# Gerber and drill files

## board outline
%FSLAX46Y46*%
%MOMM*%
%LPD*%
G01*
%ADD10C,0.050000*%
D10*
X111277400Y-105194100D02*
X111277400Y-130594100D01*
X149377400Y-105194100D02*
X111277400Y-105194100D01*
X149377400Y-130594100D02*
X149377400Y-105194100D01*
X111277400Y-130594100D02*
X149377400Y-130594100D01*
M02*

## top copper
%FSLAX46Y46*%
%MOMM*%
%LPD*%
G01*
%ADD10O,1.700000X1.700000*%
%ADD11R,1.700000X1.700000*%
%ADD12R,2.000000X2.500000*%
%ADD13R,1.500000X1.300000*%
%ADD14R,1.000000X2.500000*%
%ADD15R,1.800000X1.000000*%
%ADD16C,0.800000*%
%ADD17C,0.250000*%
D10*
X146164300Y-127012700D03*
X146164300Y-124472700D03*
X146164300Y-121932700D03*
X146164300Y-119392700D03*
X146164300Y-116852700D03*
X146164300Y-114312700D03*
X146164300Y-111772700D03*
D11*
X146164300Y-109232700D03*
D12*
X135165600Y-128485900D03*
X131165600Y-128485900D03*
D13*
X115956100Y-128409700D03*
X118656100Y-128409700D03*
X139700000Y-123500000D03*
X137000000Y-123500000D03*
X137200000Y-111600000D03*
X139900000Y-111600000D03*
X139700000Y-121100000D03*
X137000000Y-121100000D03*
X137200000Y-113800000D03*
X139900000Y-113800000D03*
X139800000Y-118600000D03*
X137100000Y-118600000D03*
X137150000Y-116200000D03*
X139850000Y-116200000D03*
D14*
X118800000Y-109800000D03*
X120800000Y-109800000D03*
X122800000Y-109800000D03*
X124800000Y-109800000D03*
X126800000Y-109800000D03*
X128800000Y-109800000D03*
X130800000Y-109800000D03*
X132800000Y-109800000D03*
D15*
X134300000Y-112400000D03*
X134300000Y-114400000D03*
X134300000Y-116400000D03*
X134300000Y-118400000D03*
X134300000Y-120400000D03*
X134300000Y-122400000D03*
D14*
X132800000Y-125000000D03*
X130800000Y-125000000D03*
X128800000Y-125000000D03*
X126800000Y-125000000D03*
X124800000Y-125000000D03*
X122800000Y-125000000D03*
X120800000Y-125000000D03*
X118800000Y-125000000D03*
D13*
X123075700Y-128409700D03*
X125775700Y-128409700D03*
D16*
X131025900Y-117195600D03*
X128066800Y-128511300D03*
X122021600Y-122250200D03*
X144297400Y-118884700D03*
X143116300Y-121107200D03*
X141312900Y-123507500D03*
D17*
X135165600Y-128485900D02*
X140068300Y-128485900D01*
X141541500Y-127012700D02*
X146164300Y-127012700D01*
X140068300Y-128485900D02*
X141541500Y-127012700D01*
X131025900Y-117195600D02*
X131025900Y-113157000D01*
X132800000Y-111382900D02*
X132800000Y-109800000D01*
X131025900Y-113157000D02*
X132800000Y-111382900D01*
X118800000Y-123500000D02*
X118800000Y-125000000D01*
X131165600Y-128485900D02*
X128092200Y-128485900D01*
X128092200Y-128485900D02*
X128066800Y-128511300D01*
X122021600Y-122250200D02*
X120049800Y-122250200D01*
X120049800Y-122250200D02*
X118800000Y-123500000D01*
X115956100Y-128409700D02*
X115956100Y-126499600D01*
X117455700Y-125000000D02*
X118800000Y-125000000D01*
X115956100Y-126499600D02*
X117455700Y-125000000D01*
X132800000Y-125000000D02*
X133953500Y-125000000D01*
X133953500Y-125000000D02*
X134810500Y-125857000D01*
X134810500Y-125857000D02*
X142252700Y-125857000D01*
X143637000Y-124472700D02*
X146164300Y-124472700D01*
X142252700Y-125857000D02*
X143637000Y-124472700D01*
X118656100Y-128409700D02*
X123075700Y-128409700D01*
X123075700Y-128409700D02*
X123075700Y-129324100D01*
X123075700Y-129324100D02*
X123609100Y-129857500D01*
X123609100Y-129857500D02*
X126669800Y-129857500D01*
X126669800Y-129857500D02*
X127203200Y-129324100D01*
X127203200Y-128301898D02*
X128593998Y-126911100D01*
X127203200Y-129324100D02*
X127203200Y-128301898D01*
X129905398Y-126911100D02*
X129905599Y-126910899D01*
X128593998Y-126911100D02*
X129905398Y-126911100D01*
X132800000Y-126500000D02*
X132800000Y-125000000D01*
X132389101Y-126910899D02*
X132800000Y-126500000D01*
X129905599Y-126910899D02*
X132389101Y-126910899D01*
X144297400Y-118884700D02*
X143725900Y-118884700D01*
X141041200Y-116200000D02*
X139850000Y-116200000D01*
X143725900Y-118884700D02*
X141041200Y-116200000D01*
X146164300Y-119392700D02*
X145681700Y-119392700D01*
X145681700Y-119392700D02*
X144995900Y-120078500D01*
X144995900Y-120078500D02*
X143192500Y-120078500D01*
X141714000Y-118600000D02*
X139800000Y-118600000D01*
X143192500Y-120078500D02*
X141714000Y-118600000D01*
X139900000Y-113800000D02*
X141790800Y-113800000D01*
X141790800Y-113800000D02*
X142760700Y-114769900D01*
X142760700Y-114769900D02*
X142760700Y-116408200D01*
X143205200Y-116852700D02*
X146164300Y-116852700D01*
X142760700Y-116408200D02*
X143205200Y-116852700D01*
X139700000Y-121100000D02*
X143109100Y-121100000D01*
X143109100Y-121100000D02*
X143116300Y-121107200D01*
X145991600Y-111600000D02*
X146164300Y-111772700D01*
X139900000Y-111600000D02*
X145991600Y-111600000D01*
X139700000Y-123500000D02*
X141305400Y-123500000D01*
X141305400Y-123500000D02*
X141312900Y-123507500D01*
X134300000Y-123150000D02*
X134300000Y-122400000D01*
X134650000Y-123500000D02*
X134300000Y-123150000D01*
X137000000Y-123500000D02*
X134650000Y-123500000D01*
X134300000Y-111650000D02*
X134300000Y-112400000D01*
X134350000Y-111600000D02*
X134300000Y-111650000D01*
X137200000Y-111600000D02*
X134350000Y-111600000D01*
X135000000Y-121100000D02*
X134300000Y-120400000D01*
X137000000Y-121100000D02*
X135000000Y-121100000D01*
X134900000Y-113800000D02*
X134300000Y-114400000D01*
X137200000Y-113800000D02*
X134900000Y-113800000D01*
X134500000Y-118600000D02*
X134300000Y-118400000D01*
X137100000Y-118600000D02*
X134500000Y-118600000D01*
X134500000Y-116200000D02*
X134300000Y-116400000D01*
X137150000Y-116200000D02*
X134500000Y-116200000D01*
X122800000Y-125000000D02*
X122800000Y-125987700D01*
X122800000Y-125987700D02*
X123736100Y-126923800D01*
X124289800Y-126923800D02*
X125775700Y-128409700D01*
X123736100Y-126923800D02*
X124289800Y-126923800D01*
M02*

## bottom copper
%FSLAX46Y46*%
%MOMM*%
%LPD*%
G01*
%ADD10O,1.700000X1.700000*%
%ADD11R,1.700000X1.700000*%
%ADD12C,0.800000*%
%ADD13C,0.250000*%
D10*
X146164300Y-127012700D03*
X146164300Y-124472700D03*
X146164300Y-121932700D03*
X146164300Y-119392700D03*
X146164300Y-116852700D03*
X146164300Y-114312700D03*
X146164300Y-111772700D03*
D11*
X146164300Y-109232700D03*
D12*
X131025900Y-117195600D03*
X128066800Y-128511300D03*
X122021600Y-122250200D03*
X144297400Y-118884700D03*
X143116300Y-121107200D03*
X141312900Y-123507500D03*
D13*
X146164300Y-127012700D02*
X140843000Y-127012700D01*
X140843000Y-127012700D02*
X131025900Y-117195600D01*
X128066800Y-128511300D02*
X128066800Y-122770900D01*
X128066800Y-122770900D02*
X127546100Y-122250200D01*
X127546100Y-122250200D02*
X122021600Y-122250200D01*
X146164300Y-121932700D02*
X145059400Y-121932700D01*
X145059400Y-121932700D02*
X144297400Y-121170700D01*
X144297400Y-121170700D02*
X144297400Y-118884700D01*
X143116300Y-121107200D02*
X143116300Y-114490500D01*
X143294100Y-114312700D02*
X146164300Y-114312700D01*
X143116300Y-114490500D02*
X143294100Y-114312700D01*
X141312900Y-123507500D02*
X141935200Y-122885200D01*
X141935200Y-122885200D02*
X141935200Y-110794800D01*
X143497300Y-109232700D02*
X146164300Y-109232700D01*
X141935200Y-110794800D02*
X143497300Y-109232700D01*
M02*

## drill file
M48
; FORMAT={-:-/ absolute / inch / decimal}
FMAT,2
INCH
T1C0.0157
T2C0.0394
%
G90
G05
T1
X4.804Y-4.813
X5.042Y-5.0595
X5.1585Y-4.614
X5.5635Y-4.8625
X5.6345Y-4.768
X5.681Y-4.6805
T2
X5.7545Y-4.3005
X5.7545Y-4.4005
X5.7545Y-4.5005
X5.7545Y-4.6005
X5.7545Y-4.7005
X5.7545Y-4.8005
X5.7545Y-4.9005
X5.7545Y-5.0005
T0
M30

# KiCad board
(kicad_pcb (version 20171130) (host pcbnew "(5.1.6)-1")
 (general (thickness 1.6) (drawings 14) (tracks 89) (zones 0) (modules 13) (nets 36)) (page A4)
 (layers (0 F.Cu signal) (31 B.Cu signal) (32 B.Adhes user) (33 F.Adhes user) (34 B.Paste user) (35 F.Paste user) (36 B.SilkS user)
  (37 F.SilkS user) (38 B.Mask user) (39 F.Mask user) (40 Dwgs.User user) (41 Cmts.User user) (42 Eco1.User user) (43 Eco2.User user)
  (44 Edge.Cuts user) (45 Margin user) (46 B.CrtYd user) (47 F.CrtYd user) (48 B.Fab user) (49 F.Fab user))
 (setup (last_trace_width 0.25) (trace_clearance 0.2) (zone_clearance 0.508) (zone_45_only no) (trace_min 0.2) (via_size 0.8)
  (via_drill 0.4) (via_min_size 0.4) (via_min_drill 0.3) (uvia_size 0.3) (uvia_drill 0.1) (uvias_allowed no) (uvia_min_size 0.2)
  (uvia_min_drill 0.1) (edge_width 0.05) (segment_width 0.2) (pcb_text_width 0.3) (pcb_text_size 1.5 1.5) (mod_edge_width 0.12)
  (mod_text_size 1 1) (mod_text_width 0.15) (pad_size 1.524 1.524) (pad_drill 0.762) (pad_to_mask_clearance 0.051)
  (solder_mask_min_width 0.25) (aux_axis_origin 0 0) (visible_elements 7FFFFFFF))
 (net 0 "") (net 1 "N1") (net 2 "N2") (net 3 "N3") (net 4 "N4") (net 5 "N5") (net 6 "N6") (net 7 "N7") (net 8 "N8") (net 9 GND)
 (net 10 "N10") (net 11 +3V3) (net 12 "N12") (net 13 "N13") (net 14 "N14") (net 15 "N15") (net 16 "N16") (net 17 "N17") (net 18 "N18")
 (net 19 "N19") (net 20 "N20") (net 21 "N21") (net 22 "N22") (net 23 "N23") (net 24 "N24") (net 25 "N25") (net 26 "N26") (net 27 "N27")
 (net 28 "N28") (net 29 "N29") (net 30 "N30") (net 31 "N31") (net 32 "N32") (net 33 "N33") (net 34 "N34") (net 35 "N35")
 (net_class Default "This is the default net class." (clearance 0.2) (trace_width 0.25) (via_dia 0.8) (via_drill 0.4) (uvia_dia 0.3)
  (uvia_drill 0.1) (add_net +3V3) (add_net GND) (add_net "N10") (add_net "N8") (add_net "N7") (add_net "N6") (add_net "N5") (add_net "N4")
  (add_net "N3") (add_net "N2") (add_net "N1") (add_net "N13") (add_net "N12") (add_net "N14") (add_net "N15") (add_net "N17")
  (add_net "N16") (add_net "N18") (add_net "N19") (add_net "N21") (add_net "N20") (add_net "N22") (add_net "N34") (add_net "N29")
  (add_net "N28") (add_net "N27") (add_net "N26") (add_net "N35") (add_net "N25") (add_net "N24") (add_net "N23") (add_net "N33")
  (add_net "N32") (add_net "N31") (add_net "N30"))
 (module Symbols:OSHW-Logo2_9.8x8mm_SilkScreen (layer B.Cu) (at 131.37388 117.3861 270)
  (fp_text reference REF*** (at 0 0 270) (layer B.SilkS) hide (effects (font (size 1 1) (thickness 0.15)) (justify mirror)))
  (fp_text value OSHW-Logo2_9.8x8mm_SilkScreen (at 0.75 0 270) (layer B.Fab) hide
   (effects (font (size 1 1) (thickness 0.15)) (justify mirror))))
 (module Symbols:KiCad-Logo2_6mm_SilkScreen (layer B.Cu) (at 119.09298 117.41404 270)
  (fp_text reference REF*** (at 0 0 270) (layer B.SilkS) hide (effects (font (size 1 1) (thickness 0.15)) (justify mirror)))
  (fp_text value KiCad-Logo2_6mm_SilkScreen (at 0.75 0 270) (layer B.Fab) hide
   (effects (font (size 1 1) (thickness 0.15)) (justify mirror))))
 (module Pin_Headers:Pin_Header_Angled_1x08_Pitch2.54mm (layer F.Cu) (at 146.1643 109.2327)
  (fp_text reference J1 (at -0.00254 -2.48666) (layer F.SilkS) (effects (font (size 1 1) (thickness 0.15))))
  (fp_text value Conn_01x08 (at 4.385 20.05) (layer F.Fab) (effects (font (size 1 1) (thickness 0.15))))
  (pad 8 thru_hole oval (at 0 17.78) (size 1.7 1.7) (drill 1) (layers *.Cu *.Mask) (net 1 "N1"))
  (pad 7 thru_hole oval (at 0 15.24) (size 1.7 1.7) (drill 1) (layers *.Cu *.Mask) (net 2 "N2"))
  (pad 6 thru_hole oval (at 0 12.7) (size 1.7 1.7) (drill 1) (layers *.Cu *.Mask) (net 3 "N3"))
  (pad 5 thru_hole oval (at 0 10.16) (size 1.7 1.7) (drill 1) (layers *.Cu *.Mask) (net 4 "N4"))
  (pad 4 thru_hole oval (at 0 7.62) (size 1.7 1.7) (drill 1) (layers *.Cu *.Mask) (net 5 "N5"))
  (pad 3 thru_hole oval (at 0 5.08) (size 1.7 1.7) (drill 1) (layers *.Cu *.Mask) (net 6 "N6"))
  (pad 2 thru_hole oval (at 0 2.54) (size 1.7 1.7) (drill 1) (layers *.Cu *.Mask) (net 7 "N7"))
  (pad 1 thru_hole rect (at 0 0) (size 1.7 1.7) (drill 1) (layers *.Cu *.Mask) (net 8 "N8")))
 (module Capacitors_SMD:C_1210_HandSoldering (layer F.Cu) (at 133.1656 128.4859)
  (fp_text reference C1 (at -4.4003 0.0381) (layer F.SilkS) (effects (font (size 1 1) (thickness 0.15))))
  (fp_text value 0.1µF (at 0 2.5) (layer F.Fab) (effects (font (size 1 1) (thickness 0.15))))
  (pad 2 smd rect (at 2 0) (size 2 2.5) (layers F.Cu F.Paste F.Mask) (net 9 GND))
  (pad 1 smd rect (at -2 0) (size 2 2.5) (layers F.Cu F.Paste F.Mask) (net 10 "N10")))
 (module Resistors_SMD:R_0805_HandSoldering (layer F.Cu) (at 117.3061 128.4097 180)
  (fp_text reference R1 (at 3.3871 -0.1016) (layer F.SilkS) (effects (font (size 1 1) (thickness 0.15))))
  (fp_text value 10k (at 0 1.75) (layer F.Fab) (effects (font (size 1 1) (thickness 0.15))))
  (pad 2 smd rect (at 1.35 0 180) (size 1.5 1.3) (layers F.Cu F.Paste F.Mask) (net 10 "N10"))
  (pad 1 smd rect (at -1.35 0 180) (size 1.5 1.3) (layers F.Cu F.Paste F.Mask) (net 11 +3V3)))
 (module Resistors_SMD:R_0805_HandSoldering (layer F.Cu) (at 138.35 123.5)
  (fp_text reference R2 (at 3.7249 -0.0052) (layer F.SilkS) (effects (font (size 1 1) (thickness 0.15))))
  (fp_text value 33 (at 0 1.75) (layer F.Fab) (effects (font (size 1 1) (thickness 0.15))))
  (pad 2 smd rect (at 1.35 0) (size 1.5 1.3) (layers F.Cu F.Paste F.Mask) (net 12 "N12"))
  (pad 1 smd rect (at -1.35 0) (size 1.5 1.3) (layers F.Cu F.Paste F.Mask) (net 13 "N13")))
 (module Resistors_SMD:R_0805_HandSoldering (layer F.Cu) (at 138.55 111.6)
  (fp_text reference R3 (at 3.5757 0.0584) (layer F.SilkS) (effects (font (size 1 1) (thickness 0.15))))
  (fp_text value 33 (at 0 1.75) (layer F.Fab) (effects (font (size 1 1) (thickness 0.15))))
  (pad 1 smd rect (at -1.35 0) (size 1.5 1.3) (layers F.Cu F.Paste F.Mask) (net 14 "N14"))
  (pad 2 smd rect (at 1.35 0) (size 1.5 1.3) (layers F.Cu F.Paste F.Mask) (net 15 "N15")))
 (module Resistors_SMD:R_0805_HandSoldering (layer F.Cu) (at 138.35 121.1)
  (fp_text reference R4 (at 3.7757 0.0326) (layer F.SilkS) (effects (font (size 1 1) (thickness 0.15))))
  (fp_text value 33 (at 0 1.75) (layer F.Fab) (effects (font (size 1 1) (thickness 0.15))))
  (pad 2 smd rect (at 1.35 0) (size 1.5 1.3) (layers F.Cu F.Paste F.Mask) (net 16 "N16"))
  (pad 1 smd rect (at -1.35 0) (size 1.5 1.3) (layers F.Cu F.Paste F.Mask) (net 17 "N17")))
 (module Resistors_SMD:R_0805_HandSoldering (layer F.Cu) (at 138.55 113.8)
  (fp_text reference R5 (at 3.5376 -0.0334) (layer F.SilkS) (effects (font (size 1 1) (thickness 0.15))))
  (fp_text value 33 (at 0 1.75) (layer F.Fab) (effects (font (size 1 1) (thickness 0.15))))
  (pad 1 smd rect (at -1.35 0) (size 1.5 1.3) (layers F.Cu F.Paste F.Mask) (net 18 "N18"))
  (pad 2 smd rect (at 1.35 0) (size 1.5 1.3) (layers F.Cu F.Paste F.Mask) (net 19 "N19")))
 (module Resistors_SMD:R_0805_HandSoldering (layer F.Cu) (at 138.45 118.6)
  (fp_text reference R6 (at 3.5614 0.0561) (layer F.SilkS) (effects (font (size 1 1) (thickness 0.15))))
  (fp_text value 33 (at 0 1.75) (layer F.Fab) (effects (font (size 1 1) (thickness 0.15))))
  (pad 2 smd rect (at 1.35 0) (size 1.5 1.3) (layers F.Cu F.Paste F.Mask) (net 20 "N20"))
  (pad 1 smd rect (at -1.35 0) (size 1.5 1.3) (layers F.Cu F.Paste F.Mask) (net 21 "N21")))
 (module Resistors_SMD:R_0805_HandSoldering (layer F.Cu) (at 138.5 116.2)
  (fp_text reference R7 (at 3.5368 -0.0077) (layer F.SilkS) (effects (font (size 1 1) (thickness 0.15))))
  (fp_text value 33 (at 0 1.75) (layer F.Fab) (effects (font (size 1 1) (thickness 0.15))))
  (pad 1 smd rect (at -1.35 0) (size 1.5 1.3) (layers F.Cu F.Paste F.Mask) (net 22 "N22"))
  (pad 2 smd rect (at 1.35 0) (size 1.5 1.3) (layers F.Cu F.Paste F.Mask) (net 7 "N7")))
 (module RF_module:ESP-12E (layer F.Cu) (at 122.3 117.4 90)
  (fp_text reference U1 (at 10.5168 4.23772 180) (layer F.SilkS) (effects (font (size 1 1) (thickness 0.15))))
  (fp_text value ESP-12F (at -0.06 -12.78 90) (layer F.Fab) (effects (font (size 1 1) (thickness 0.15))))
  (pad 22 smd rect (at 7.6 -3.5 90) (size 2.5 1) (layers F.Cu F.Paste F.Mask) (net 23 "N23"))
  (pad 21 smd rect (at 7.6 -1.5 90) (size 2.5 1) (layers F.Cu F.Paste F.Mask) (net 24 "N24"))
  (pad 20 smd rect (at 7.6 0.5 90) (size 2.5 1) (layers F.Cu F.Paste F.Mask) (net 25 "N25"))
  (pad 19 smd rect (at 7.6 2.5 90) (size 2.5 1) (layers F.Cu F.Paste F.Mask) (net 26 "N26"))
  (pad 18 smd rect (at 7.6 4.5 90) (size 2.5 1) (layers F.Cu F.Paste F.Mask) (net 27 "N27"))
  (pad 17 smd rect (at 7.6 6.5 90) (size 2.5 1) (layers F.Cu F.Paste F.Mask) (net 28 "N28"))
  (pad 16 smd rect (at 7.6 8.5 90) (size 2.5 1) (layers F.Cu F.Paste F.Mask) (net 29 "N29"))
  (pad 15 smd rect (at 7.6 10.5 90) (size 2.5 1) (layers F.Cu F.Paste F.Mask) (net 9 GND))
  (pad 14 smd rect (at 5 12 90) (size 1 1.8) (layers F.Cu F.Paste F.Mask) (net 14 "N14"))
  (pad 13 smd rect (at 3 12 90) (size 1 1.8) (layers F.Cu F.Paste F.Mask) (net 18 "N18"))
  (pad 12 smd rect (at 1 12 90) (size 1 1.8) (layers F.Cu F.Paste F.Mask) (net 22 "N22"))
  (pad 11 smd rect (at -1 12 90) (size 1 1.8) (layers F.Cu F.Paste F.Mask) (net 21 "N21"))
  (pad 10 smd rect (at -3 12 90) (size 1 1.8) (layers F.Cu F.Paste F.Mask) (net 17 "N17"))
  (pad 9 smd rect (at -5 12 90) (size 1 1.8) (layers F.Cu F.Paste F.Mask) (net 13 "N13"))
  (pad 8 smd rect (at -7.6 10.5 90) (size 2.5 1) (layers F.Cu F.Paste F.Mask) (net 11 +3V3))
  (pad 7 smd rect (at -7.6 8.5 90) (size 2.5 1) (layers F.Cu F.Paste F.Mask) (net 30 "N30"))
  (pad 6 smd rect (at -7.6 6.5 90) (size 2.5 1) (layers F.Cu F.Paste F.Mask) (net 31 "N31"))
  (pad 5 smd rect (at -7.6 4.5 90) (size 2.5 1) (layers F.Cu F.Paste F.Mask) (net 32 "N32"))
  (pad 4 smd rect (at -7.6 2.5 90) (size 2.5 1) (layers F.Cu F.Paste F.Mask) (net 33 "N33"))
  (pad 3 smd rect (at -7.6 0.5 90) (size 2.5 1) (layers F.Cu F.Paste F.Mask) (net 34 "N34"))
  (pad 2 smd rect (at -7.6 -1.5 90) (size 2.5 1) (layers F.Cu F.Paste F.Mask) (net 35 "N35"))
  (pad 1 smd rect (at -7.6 -3.5 90) (size 2.5 1) (layers F.Cu F.Paste F.Mask) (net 10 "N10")))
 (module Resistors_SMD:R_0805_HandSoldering (layer F.Cu) (at 124.4257 128.4097 180)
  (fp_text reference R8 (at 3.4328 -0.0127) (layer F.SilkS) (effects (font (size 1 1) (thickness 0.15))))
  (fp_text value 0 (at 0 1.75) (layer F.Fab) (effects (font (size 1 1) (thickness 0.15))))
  (pad 2 smd rect (at 1.35 0 180) (size 1.5 1.3) (layers F.Cu F.Paste F.Mask) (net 11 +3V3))
  (pad 1 smd rect (at -1.35 0 180) (size 1.5 1.3) (layers F.Cu F.Paste F.Mask) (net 34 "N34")))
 (gr_line (start 111.2774 105.1941) (end 111.2774 130.5941) (layer Edge.Cuts) (width 0.05))
 (gr_line (start 149.3774 105.1941) (end 111.2774 105.1941) (layer Edge.Cuts) (width 0.05))
 (gr_line (start 149.3774 130.5941) (end 149.3774 105.1941) (layer Edge.Cuts) (width 0.05))
 (gr_line (start 111.2774 130.5941) (end 149.3774 130.5941) (layer Edge.Cuts) (width 0.05))
 (segment (start 135.1656 128.4859) (end 140.0683 128.4859) (width 0.25) (layer F.Cu) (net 9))
 (segment (start 141.5415 127.0127) (end 146.1643 127.0127) (width 0.25) (layer F.Cu) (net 9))
 (segment (start 140.0683 128.4859) (end 141.5415 127.0127) (width 0.25) (layer F.Cu) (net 9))
 (segment (start 146.1643 127.0127) (end 140.843 127.0127) (width 0.25) (layer B.Cu) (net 9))
 (via (at 131.0259 117.1956) (size 0.8) (drill 0.4) (layers F.Cu B.Cu) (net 9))
 (segment (start 140.843 127.0127) (end 131.0259 117.1956) (width 0.25) (layer B.Cu) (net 9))
 (segment (start 131.0259 117.1956) (end 131.0259 113.157) (width 0.25) (layer F.Cu) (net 9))
 (segment (start 132.8 111.3829) (end 132.8 109.8) (width 0.25) (layer F.Cu) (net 9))
 (segment (start 131.0259 113.157) (end 132.8 111.3829) (width 0.25) (layer F.Cu) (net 9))
 (segment (start 128.0668 128.5113) (end 128.0668 122.7709) (width 0.25) (layer B.Cu) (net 10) (status 1000000))
 (segment (start 118.8 123.5) (end 118.8 125) (width 0.25) (layer F.Cu) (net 10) (status 1000000))
 (segment (start 131.1656 128.4859) (end 128.0922 128.4859) (width 0.25) (layer F.Cu) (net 10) (status 1000000))
 (segment (start 128.0668 122.7709) (end 127.5461 122.2502) (width 0.25) (layer B.Cu) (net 10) (status 1000000))
 (segment (start 127.5461 122.2502) (end 122.0216 122.2502) (width 0.25) (layer B.Cu) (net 10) (status 1000000))
 (segment (start 128.0922 128.4859) (end 128.0668 128.5113) (width 0.25) (layer F.Cu) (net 10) (status 1000000))
 (segment (start 122.0216 122.2502) (end 120.0498 122.2502) (width 0.25) (layer F.Cu) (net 10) (status 1000000))
 (segment (start 120.0498 122.2502) (end 118.8 123.5) (width 0.25) (layer F.Cu) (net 10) (status 1000000))
 (via (at 128.0668 128.5113) (size 0.8) (drill 0.4) (layers F.Cu B.Cu) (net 10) (status 1000000))
 (via (at 122.0216 122.2502) (size 0.8) (drill 0.4) (layers F.Cu B.Cu) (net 10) (status 1000000))
 (segment (start 115.9561 128.4097) (end 115.9561 126.4996) (width 0.25) (layer F.Cu) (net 10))
 (segment (start 117.4557 125) (end 118.8 125) (width 0.25) (layer F.Cu) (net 10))
 (segment (start 115.9561 126.4996) (end 117.4557 125) (width 0.25) (layer F.Cu) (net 10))
 (segment (start 132.8 125) (end 133.9535 125) (width 0.25) (layer F.Cu) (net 11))
 (segment (start 133.9535 125) (end 134.8105 125.857) (width 0.25) (layer F.Cu) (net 11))
 (segment (start 134.8105 125.857) (end 142.2527 125.857) (width 0.25) (layer F.Cu) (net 11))
 (segment (start 143.637 124.4727) (end 146.1643 124.4727) (width 0.25) (layer F.Cu) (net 11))
 (segment (start 142.2527 125.857) (end 143.637 124.4727) (width 0.25) (layer F.Cu) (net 11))
 (segment (start 118.6561 128.4097) (end 123.0757 128.4097) (width 0.25) (layer F.Cu) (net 11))
 (segment (start 123.0757 128.4097) (end 123.0757 129.3241) (width 0.25) (layer F.Cu) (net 11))
 (segment (start 123.0757 129.3241) (end 123.6091 129.8575) (width 0.25) (layer F.Cu) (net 11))
 (segment (start 123.6091 129.8575) (end 126.6698 129.8575) (width 0.25) (layer F.Cu) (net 11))
 (segment (start 126.6698 129.8575) (end 127.2032 129.3241) (width 0.25) (layer F.Cu) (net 11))
 (segment (start 127.2032 128.301898) (end 128.593998 126.9111) (width 0.25) (layer F.Cu) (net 11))
 (segment (start 127.2032 129.3241) (end 127.2032 128.301898) (width 0.25) (layer F.Cu) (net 11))
 (segment (start 129.905398 126.9111) (end 129.905599 126.910899) (width 0.25) (layer F.Cu) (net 11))
 (segment (start 128.593998 126.9111) (end 129.905398 126.9111) (width 0.25) (layer F.Cu) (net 11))
 (segment (start 132.8 126.5) (end 132.8 125) (width 0.25) (layer F.Cu) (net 11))
 (segment (start 132.389101 126.910899) (end 132.8 126.5) (width 0.25) (layer F.Cu) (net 11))
 (segment (start 129.905599 126.910899) (end 132.389101 126.910899) (width 0.25) (layer F.Cu) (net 11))
 (segment (start 146.1643 121.9327) (end 145.0594 121.9327) (width 0.25) (layer B.Cu) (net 3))
 (via (at 144.2974 118.8847) (size 0.8) (drill 0.4) (layers F.Cu B.Cu) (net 3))
 (segment (start 145.0594 121.9327) (end 144.2974 121.1707) (width 0.25) (layer B.Cu) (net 3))
 (segment (start 144.2974 121.1707) (end 144.2974 118.8847) (width 0.25) (layer B.Cu) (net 3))
 (segment (start 144.2974 118.8847) (end 143.7259 118.8847) (width 0.25) (layer F.Cu) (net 3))
 (segment (start 141.0412 116.2) (end 139.85 116.2) (width 0.25) (layer F.Cu) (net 3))
 (segment (start 143.7259 118.8847) (end 141.0412 116.2) (width 0.25) (layer F.Cu) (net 3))
 (segment (start 146.1643 119.3927) (end 145.6817 119.3927) (width 0.25) (layer F.Cu) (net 4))
 (segment (start 145.6817 119.3927) (end 144.9959 120.0785) (width 0.25) (layer F.Cu) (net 4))
 (segment (start 144.9959 120.0785) (end 143.1925 120.0785) (width 0.25) (layer F.Cu) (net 4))
 (segment (start 141.714 118.6) (end 139.8 118.6) (width 0.25) (layer F.Cu) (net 4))
 (segment (start 143.1925 120.0785) (end 141.714 118.6) (width 0.25) (layer F.Cu) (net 4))
 (segment (start 139.9 113.8) (end 141.7908 113.8) (width 0.25) (layer F.Cu) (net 5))
 (segment (start 141.7908 113.8) (end 142.7607 114.7699) (width 0.25) (layer F.Cu) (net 5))
 (segment (start 142.7607 114.7699) (end 142.7607 116.4082) (width 0.25) (layer F.Cu) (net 5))
 (segment (start 143.2052 116.8527) (end 146.1643 116.8527) (width 0.25) (layer F.Cu) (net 5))
 (segment (start 142.7607 116.4082) (end 143.2052 116.8527) (width 0.25) (layer F.Cu) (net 5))
 (via (at 143.1163 121.1072) (size 0.8) (drill 0.4) (layers F.Cu B.Cu) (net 6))
 (segment (start 139.7 121.1) (end 143.1091 121.1) (width 0.25) (layer F.Cu) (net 6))
 (segment (start 143.1091 121.1) (end 143.1163 121.1072) (width 0.25) (layer F.Cu) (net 6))
 (segment (start 143.1163 121.1072) (end 143.1163 114.4905) (width 0.25) (layer B.Cu) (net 6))
 (segment (start 143.2941 114.3127) (end 146.1643 114.3127) (width 0.25) (layer B.Cu) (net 6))
 (segment (start 143.1163 114.4905) (end 143.2941 114.3127) (width 0.25) (layer B.Cu) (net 6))
 (segment (start 145.9916 111.6) (end 146.1643 111.7727) (width 0.25) (layer F.Cu) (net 7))
 (segment (start 139.9 111.6) (end 145.9916 111.6) (width 0.25) (layer F.Cu) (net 7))
 (via (at 141.3129 123.5075) (size 0.8) (drill 0.4) (layers F.Cu B.Cu) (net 8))
 (segment (start 139.7 123.5) (end 141.3054 123.5) (width 0.25) (layer F.Cu) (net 8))
 (segment (start 141.3054 123.5) (end 141.3129 123.5075) (width 0.25) (layer F.Cu) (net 8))
 (segment (start 141.3129 123.5075) (end 141.9352 122.8852) (width 0.25) (layer B.Cu) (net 8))
 (segment (start 141.9352 122.8852) (end 141.9352 110.7948) (width 0.25) (layer B.Cu) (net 8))
 (segment (start 143.4973 109.2327) (end 146.1643 109.2327) (width 0.25) (layer B.Cu) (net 8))
 (segment (start 141.9352 110.7948) (end 143.4973 109.2327) (width 0.25) (layer B.Cu) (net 8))
 (segment (start 134.3 123.15) (end 134.3 122.4) (width 0.25) (layer F.Cu) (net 13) (status 20))
 (segment (start 134.65 123.5) (end 134.3 123.15) (width 0.25) (layer F.Cu) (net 13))
 (segment (start 137 123.5) (end 134.65 123.5) (width 0.25) (layer F.Cu) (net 13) (status 10))
 (segment (start 134.3 111.65) (end 134.3 112.4) (width 0.25) (layer F.Cu) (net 14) (status 20))
 (segment (start 134.35 111.6) (end 134.3 111.65) (width 0.25) (layer F.Cu) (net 14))
 (segment (start 137.2 111.6) (end 134.35 111.6) (width 0.25) (layer F.Cu) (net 14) (status 10))
 (segment (start 135 121.1) (end 134.3 120.4) (width 0.25) (layer F.Cu) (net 17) (status 20))
 (segment (start 137 121.1) (end 135 121.1) (width 0.25) (layer F.Cu) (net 17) (status 10))
 (segment (start 134.9 113.8) (end 134.3 114.4) (width 0.25) (layer F.Cu) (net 18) (status 20))
 (segment (start 137.2 113.8) (end 134.9 113.8) (width 0.25) (layer F.Cu) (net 18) (status 10))
 (segment (start 134.5 118.6) (end 134.3 118.4) (width 0.25) (layer F.Cu) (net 21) (status 30))
 (segment (start 137.1 118.6) (end 134.5 118.6) (width 0.25) (layer F.Cu) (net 21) (status 30))
 (segment (start 134.5 116.2) (end 134.3 116.4) (width 0.25) (layer F.Cu) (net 22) (status 30))
 (segment (start 137.15 116.2) (end 134.5 116.2) (width 0.25) (layer F.Cu) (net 22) (status 30))
 (segment (start 122.8 125) (end 122.8 125.9877) (width 0.25) (layer F.Cu) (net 34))
 (segment (start 122.8 125.9877) (end 123.7361 126.9238) (width 0.25) (layer F.Cu) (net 34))
 (segment (start 124.2898 126.9238) (end 125.7757 128.4097) (width 0.25) (layer F.Cu) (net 34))
 (segment (start 123.7361 126.9238) (end 124.2898 126.9238) (width 0.25) (layer F.Cu) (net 34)))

